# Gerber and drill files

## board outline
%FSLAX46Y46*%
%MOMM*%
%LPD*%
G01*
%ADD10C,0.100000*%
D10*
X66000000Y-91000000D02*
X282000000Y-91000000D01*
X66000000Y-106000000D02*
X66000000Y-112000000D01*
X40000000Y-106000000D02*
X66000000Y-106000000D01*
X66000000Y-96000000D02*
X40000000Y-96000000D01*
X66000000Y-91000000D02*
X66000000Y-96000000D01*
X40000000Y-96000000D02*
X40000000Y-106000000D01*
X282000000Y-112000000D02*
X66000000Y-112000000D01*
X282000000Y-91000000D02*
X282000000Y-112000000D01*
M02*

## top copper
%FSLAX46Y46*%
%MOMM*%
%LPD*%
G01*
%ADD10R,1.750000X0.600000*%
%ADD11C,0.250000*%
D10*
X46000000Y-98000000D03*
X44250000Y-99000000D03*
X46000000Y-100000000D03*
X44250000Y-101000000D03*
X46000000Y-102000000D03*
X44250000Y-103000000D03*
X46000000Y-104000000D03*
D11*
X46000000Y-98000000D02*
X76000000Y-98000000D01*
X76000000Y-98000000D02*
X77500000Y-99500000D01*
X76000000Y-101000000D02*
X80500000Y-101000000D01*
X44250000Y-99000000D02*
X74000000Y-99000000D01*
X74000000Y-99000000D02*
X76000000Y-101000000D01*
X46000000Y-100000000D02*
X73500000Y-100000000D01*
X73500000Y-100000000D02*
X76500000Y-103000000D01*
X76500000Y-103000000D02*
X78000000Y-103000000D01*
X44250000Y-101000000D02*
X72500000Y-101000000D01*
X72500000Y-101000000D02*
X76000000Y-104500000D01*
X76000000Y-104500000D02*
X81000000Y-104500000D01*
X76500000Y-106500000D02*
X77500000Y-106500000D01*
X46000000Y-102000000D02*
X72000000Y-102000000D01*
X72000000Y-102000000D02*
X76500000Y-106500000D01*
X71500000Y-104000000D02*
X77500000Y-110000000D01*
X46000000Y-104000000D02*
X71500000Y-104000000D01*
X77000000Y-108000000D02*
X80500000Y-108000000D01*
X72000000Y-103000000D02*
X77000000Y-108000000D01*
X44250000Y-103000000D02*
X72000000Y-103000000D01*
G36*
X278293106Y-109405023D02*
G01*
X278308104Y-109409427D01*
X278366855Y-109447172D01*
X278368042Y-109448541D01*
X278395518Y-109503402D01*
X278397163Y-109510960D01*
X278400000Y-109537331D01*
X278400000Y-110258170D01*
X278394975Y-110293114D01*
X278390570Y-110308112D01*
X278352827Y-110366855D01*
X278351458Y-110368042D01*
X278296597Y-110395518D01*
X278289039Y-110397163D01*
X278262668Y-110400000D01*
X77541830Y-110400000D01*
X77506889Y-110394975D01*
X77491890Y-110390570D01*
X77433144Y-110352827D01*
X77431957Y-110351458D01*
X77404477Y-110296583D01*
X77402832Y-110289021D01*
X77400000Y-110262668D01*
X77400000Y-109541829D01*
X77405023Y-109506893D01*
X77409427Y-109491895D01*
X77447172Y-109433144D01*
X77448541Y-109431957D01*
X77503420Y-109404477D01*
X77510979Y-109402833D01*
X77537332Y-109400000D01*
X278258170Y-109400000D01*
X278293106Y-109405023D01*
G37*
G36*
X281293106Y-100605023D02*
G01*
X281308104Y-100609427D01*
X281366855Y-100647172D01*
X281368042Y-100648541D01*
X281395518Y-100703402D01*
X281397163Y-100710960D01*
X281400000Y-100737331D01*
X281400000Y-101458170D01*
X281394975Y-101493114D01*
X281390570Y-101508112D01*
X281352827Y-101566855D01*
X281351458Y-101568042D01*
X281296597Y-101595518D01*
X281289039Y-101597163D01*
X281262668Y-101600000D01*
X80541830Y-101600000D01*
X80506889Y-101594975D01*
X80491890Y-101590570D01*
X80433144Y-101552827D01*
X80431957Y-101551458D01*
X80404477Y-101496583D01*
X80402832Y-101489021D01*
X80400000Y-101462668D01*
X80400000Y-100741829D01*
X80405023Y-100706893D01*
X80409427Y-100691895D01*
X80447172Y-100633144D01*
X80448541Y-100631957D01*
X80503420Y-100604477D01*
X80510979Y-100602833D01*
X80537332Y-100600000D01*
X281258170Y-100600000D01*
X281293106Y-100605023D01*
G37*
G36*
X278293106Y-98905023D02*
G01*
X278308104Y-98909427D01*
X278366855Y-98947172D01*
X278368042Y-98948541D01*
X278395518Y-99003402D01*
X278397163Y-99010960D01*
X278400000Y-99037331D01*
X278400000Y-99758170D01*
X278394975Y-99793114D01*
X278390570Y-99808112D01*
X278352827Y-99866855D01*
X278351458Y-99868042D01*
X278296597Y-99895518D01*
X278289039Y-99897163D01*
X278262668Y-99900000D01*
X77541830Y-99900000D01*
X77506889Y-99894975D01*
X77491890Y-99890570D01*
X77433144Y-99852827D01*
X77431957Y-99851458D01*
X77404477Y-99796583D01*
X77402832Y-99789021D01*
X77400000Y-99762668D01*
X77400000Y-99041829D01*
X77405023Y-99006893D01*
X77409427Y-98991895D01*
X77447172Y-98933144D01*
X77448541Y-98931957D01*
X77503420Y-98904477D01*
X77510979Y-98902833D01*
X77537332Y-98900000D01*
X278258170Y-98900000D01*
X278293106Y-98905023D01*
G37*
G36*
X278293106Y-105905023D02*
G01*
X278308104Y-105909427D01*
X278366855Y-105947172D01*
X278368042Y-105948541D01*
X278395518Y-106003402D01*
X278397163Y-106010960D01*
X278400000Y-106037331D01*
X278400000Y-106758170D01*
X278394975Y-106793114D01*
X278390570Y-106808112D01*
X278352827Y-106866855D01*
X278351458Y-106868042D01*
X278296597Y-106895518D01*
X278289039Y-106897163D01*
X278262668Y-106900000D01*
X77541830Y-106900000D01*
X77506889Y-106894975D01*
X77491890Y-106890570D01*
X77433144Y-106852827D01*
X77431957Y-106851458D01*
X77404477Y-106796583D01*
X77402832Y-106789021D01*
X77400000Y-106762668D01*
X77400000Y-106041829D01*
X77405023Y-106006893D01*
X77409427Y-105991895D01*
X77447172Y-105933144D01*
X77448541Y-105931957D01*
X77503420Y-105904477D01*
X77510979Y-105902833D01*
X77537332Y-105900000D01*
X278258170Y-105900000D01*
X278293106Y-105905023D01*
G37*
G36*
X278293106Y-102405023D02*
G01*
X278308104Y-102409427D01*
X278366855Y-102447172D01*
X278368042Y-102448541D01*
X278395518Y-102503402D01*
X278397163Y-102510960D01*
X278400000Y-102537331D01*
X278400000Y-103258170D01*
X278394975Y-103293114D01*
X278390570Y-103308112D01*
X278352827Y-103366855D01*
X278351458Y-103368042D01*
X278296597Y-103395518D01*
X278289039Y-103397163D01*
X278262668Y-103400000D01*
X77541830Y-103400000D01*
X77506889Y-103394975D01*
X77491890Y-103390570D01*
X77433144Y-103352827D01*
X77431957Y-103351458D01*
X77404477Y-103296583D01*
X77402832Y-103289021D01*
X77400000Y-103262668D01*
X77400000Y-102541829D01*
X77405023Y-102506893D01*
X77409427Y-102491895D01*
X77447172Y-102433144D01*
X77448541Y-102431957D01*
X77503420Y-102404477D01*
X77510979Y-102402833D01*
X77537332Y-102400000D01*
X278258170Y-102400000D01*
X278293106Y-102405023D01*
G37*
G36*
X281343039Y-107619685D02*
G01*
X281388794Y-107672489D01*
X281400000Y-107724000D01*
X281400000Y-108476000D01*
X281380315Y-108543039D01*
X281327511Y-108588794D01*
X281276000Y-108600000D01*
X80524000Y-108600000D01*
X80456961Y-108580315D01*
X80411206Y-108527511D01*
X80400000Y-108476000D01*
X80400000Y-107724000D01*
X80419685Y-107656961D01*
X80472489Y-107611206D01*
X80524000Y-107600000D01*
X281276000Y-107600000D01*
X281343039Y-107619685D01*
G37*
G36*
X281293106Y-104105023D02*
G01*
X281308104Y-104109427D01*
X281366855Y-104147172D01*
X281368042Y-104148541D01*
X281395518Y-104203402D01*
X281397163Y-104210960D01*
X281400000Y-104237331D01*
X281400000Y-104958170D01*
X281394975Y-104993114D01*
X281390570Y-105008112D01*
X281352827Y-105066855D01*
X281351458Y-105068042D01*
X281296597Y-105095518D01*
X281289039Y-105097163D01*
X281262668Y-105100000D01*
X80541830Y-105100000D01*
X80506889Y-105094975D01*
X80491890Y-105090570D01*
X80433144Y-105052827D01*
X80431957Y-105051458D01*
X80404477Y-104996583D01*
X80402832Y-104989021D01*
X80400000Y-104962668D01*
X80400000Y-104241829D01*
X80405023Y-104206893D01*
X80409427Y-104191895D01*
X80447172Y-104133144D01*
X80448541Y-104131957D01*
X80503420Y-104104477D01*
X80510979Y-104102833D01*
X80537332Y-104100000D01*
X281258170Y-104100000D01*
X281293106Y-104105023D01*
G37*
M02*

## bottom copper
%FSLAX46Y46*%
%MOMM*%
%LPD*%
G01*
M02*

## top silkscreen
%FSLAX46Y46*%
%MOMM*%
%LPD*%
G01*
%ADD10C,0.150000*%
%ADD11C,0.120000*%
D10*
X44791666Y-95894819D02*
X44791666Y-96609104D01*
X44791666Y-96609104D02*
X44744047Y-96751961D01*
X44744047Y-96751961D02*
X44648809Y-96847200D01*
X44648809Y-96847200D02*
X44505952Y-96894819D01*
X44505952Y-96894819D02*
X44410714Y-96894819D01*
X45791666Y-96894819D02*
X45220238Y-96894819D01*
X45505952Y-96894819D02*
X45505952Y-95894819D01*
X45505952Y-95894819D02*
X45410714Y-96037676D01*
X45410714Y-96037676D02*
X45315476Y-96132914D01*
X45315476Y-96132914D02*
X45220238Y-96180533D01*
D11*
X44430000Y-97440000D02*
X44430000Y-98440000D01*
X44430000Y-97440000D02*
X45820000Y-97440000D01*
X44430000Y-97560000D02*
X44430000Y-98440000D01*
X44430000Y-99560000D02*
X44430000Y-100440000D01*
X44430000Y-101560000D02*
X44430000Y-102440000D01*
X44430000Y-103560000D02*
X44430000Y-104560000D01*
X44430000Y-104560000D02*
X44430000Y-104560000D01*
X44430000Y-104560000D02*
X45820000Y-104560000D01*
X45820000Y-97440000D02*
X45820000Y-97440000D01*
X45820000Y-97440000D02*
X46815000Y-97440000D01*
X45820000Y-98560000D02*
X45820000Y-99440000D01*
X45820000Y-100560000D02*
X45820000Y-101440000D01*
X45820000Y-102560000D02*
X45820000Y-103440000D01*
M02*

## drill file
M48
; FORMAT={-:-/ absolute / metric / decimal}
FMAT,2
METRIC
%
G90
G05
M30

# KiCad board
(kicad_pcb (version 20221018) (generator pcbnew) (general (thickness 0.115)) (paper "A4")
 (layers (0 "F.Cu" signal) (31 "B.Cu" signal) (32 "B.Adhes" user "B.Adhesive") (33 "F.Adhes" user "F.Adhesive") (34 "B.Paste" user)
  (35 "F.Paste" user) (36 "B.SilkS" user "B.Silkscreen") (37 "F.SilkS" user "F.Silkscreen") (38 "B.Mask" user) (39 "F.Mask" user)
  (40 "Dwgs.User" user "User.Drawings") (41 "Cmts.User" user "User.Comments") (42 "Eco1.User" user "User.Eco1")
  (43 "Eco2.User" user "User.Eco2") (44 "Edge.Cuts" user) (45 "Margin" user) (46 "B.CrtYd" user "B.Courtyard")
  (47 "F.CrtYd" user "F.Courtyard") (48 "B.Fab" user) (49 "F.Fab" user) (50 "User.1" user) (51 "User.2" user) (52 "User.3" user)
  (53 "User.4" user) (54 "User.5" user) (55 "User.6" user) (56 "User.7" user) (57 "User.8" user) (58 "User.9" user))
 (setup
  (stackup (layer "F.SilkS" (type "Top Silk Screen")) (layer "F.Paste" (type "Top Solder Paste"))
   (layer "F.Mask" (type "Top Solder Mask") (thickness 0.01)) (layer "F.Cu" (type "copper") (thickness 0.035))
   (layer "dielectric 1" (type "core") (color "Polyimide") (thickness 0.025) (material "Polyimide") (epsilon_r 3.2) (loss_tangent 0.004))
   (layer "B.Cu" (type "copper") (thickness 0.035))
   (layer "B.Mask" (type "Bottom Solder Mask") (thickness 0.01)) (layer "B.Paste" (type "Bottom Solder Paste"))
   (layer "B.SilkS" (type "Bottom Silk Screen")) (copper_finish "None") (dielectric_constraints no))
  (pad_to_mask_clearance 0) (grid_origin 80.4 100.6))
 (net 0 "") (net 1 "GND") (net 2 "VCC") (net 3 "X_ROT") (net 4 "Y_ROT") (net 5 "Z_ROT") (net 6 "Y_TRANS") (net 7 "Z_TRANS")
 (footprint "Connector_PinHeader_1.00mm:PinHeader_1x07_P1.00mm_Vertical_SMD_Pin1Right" (layer "F.Cu") (at 45.125 101)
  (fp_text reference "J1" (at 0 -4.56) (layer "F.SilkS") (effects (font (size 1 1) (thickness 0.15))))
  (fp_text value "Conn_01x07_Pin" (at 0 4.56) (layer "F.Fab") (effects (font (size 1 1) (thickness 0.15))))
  (fp_line (start -0.695 -3.56) (end -0.695 -2.56) (stroke (width 0.12) (type solid)) (layer "F.SilkS"))
  (fp_line (start -0.695 -3.56) (end 0.695 -3.56) (stroke (width 0.12) (type solid)) (layer "F.SilkS"))
  (fp_line (start -0.695 -3.44) (end -0.695 -2.56) (stroke (width 0.12) (type solid)) (layer "F.SilkS"))
  (fp_line (start -0.695 -1.44) (end -0.695 -0.56) (stroke (width 0.12) (type solid)) (layer "F.SilkS"))
  (fp_line (start -0.695 0.56) (end -0.695 1.44) (stroke (width 0.12) (type solid)) (layer "F.SilkS"))
  (fp_line (start -0.695 2.56) (end -0.695 3.56) (stroke (width 0.12) (type solid)) (layer "F.SilkS"))
  (fp_line (start -0.695 3.56) (end -0.695 3.56) (stroke (width 0.12) (type solid)) (layer "F.SilkS"))
  (fp_line (start -0.695 3.56) (end 0.695 3.56) (stroke (width 0.12) (type solid)) (layer "F.SilkS"))
  (fp_line (start 0.695 -3.56) (end 0.695 -3.56) (stroke (width 0.12) (type solid)) (layer "F.SilkS"))
  (fp_line (start 0.695 -3.56) (end 1.69 -3.56) (stroke (width 0.12) (type solid)) (layer "F.SilkS"))
  (fp_line (start 0.695 -2.44) (end 0.695 -1.56) (stroke (width 0.12) (type solid)) (layer "F.SilkS"))
  (fp_line (start 0.695 -0.44) (end 0.695 0.44) (stroke (width 0.12) (type solid)) (layer "F.SilkS"))
  (fp_line (start 0.695 1.56) (end 0.695 2.44) (stroke (width 0.12) (type solid)) (layer "F.SilkS"))
  (pad "1" smd rect (at 0.875 -3) (size 1.75 0.6) (layers "F.Cu" "F.Paste" "F.Mask") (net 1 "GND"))
  (pad "2" smd rect (at -0.875 -2) (size 1.75 0.6) (layers "F.Cu" "F.Paste" "F.Mask") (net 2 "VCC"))
  (pad "3" smd rect (at 0.875 -1) (size 1.75 0.6) (layers "F.Cu" "F.Paste" "F.Mask") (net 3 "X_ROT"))
  (pad "4" smd rect (at -0.875 0) (size 1.75 0.6) (layers "F.Cu" "F.Paste" "F.Mask") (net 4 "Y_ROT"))
  (pad "5" smd rect (at 0.875 1) (size 1.75 0.6) (layers "F.Cu" "F.Paste" "F.Mask") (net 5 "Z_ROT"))
  (pad "6" smd rect (at -0.875 2) (size 1.75 0.6) (layers "F.Cu" "F.Paste" "F.Mask") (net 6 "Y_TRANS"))
  (pad "7" smd rect (at 0.875 3) (size 1.75 0.6) (layers "F.Cu" "F.Paste" "F.Mask") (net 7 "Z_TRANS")))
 (gr_line (start 66 91) (end 282 91) (stroke (width 0.1) (type default)) (layer "Edge.Cuts"))
 (gr_line (start 66 106) (end 66 112) (stroke (width 0.1) (type default)) (layer "Edge.Cuts"))
 (gr_line (start 40 106) (end 66 106) (stroke (width 0.1) (type default)) (layer "Edge.Cuts"))
 (gr_line (start 66 96) (end 40 96) (stroke (width 0.1) (type default)) (layer "Edge.Cuts"))
 (gr_line (start 66 91) (end 66 96) (stroke (width 0.1) (type default)) (layer "Edge.Cuts"))
 (gr_line (start 40 96) (end 40 106) (stroke (width 0.1) (type default)) (layer "Edge.Cuts"))
 (gr_line (start 282 112) (end 66 112) (stroke (width 0.1) (type default)) (layer "Edge.Cuts"))
 (gr_line (start 282 91) (end 282 112) (stroke (width 0.1) (type default)) (layer "Edge.Cuts"))
 (segment (start 46 98) (end 76 98) (width 0.25) (layer "F.Cu") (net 1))
 (segment (start 76 98) (end 77.5 99.5) (width 0.25) (layer "F.Cu") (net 1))
 (segment (start 76 101) (end 80.5 101) (width 0.25) (layer "F.Cu") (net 2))
 (segment (start 44.25 99) (end 74 99) (width 0.25) (layer "F.Cu") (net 2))
 (segment (start 74 99) (end 76 101) (width 0.25) (layer "F.Cu") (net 2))
 (segment (start 46 100) (end 73.5 100) (width 0.25) (layer "F.Cu") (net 3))
 (segment (start 73.5 100) (end 76.5 103) (width 0.25) (layer "F.Cu") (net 3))
 (segment (start 76.5 103) (end 78 103) (width 0.25) (layer "F.Cu") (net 3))
 (segment (start 44.25 101) (end 72.5 101) (width 0.25) (layer "F.Cu") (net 4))
 (segment (start 72.5 101) (end 76 104.5) (width 0.25) (layer "F.Cu") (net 4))
 (segment (start 76 104.5) (end 81 104.5) (width 0.25) (layer "F.Cu") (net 4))
 (segment (start 76.5 106.5) (end 77.5 106.5) (width 0.25) (layer "F.Cu") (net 5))
 (segment (start 46 102) (end 72 102) (width 0.25) (layer "F.Cu") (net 5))
 (segment (start 72 102) (end 76.5 106.5) (width 0.25) (layer "F.Cu") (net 5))
 (segment (start 71.5 104) (end 77.5 110) (width 0.25) (layer "F.Cu") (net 7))
 (segment (start 46 104) (end 71.5 104) (width 0.25) (layer "F.Cu") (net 7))
 (segment (start 77 108) (end 80.5 108) (width 0.25) (layer "F.Cu") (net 6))
 (segment (start 72 103) (end 77 108) (width 0.25) (layer "F.Cu") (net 6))
 (segment (start 44.25 103) (end 72 103) (width 0.25) (layer "F.Cu") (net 6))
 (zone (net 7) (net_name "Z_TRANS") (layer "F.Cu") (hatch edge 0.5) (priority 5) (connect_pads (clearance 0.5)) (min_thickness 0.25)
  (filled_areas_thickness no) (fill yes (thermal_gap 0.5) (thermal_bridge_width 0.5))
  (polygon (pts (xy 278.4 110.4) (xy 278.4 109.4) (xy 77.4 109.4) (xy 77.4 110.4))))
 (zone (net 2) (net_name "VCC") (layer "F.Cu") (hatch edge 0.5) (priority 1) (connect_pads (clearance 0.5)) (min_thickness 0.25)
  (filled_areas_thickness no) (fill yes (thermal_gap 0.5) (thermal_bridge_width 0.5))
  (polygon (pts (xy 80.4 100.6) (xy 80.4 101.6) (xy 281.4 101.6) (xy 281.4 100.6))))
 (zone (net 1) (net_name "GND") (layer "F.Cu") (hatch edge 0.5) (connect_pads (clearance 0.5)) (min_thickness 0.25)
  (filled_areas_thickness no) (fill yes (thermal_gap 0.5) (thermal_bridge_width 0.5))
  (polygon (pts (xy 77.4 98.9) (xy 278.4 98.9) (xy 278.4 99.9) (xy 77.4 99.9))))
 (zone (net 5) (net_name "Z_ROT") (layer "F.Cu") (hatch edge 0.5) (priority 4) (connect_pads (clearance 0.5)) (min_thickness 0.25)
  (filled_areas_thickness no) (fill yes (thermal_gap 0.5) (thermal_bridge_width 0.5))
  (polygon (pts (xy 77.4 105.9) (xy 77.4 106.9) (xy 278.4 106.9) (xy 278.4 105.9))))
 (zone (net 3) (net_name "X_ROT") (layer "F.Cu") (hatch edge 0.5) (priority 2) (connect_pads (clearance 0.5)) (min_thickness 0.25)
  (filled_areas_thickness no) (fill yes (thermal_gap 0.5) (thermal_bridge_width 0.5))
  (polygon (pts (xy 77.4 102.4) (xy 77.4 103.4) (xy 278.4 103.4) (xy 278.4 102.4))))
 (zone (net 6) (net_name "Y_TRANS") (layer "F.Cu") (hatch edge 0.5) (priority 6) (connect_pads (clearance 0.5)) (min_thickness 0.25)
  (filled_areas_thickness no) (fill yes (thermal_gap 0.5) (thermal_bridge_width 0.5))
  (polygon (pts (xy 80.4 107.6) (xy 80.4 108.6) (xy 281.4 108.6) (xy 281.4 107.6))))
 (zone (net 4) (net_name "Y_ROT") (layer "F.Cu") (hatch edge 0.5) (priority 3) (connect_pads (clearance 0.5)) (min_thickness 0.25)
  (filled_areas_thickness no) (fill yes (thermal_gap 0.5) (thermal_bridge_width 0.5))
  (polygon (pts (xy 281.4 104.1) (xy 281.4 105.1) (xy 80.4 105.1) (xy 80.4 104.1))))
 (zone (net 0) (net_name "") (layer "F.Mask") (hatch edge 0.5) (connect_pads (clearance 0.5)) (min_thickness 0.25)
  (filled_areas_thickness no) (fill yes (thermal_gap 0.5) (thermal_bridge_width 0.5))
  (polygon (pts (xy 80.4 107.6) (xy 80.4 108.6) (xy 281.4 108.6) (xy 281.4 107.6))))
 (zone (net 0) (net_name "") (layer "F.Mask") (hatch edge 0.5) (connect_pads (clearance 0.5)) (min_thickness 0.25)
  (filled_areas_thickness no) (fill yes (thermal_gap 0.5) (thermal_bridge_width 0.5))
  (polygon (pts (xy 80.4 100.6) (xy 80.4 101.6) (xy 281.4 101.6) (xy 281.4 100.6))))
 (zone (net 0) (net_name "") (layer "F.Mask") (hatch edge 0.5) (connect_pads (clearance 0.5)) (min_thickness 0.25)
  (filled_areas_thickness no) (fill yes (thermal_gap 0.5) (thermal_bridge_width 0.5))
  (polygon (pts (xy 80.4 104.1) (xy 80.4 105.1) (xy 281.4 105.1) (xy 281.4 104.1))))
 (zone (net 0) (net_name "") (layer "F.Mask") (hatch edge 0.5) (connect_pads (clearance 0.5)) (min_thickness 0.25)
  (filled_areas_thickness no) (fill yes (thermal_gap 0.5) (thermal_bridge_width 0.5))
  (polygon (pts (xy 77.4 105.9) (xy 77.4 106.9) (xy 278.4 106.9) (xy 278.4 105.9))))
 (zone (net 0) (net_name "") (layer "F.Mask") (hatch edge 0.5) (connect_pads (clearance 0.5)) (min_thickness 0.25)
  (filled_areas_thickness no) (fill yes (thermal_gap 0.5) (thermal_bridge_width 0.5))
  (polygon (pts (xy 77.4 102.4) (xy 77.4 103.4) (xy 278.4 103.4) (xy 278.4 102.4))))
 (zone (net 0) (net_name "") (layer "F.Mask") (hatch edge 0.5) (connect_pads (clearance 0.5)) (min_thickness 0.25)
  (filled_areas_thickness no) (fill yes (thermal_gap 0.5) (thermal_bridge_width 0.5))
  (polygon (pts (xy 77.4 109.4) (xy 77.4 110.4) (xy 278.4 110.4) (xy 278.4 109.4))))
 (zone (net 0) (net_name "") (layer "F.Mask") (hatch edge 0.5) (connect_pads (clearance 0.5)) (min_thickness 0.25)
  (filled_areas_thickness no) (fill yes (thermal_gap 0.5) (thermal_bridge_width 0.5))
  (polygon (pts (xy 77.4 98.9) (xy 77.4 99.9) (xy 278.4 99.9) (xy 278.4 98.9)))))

